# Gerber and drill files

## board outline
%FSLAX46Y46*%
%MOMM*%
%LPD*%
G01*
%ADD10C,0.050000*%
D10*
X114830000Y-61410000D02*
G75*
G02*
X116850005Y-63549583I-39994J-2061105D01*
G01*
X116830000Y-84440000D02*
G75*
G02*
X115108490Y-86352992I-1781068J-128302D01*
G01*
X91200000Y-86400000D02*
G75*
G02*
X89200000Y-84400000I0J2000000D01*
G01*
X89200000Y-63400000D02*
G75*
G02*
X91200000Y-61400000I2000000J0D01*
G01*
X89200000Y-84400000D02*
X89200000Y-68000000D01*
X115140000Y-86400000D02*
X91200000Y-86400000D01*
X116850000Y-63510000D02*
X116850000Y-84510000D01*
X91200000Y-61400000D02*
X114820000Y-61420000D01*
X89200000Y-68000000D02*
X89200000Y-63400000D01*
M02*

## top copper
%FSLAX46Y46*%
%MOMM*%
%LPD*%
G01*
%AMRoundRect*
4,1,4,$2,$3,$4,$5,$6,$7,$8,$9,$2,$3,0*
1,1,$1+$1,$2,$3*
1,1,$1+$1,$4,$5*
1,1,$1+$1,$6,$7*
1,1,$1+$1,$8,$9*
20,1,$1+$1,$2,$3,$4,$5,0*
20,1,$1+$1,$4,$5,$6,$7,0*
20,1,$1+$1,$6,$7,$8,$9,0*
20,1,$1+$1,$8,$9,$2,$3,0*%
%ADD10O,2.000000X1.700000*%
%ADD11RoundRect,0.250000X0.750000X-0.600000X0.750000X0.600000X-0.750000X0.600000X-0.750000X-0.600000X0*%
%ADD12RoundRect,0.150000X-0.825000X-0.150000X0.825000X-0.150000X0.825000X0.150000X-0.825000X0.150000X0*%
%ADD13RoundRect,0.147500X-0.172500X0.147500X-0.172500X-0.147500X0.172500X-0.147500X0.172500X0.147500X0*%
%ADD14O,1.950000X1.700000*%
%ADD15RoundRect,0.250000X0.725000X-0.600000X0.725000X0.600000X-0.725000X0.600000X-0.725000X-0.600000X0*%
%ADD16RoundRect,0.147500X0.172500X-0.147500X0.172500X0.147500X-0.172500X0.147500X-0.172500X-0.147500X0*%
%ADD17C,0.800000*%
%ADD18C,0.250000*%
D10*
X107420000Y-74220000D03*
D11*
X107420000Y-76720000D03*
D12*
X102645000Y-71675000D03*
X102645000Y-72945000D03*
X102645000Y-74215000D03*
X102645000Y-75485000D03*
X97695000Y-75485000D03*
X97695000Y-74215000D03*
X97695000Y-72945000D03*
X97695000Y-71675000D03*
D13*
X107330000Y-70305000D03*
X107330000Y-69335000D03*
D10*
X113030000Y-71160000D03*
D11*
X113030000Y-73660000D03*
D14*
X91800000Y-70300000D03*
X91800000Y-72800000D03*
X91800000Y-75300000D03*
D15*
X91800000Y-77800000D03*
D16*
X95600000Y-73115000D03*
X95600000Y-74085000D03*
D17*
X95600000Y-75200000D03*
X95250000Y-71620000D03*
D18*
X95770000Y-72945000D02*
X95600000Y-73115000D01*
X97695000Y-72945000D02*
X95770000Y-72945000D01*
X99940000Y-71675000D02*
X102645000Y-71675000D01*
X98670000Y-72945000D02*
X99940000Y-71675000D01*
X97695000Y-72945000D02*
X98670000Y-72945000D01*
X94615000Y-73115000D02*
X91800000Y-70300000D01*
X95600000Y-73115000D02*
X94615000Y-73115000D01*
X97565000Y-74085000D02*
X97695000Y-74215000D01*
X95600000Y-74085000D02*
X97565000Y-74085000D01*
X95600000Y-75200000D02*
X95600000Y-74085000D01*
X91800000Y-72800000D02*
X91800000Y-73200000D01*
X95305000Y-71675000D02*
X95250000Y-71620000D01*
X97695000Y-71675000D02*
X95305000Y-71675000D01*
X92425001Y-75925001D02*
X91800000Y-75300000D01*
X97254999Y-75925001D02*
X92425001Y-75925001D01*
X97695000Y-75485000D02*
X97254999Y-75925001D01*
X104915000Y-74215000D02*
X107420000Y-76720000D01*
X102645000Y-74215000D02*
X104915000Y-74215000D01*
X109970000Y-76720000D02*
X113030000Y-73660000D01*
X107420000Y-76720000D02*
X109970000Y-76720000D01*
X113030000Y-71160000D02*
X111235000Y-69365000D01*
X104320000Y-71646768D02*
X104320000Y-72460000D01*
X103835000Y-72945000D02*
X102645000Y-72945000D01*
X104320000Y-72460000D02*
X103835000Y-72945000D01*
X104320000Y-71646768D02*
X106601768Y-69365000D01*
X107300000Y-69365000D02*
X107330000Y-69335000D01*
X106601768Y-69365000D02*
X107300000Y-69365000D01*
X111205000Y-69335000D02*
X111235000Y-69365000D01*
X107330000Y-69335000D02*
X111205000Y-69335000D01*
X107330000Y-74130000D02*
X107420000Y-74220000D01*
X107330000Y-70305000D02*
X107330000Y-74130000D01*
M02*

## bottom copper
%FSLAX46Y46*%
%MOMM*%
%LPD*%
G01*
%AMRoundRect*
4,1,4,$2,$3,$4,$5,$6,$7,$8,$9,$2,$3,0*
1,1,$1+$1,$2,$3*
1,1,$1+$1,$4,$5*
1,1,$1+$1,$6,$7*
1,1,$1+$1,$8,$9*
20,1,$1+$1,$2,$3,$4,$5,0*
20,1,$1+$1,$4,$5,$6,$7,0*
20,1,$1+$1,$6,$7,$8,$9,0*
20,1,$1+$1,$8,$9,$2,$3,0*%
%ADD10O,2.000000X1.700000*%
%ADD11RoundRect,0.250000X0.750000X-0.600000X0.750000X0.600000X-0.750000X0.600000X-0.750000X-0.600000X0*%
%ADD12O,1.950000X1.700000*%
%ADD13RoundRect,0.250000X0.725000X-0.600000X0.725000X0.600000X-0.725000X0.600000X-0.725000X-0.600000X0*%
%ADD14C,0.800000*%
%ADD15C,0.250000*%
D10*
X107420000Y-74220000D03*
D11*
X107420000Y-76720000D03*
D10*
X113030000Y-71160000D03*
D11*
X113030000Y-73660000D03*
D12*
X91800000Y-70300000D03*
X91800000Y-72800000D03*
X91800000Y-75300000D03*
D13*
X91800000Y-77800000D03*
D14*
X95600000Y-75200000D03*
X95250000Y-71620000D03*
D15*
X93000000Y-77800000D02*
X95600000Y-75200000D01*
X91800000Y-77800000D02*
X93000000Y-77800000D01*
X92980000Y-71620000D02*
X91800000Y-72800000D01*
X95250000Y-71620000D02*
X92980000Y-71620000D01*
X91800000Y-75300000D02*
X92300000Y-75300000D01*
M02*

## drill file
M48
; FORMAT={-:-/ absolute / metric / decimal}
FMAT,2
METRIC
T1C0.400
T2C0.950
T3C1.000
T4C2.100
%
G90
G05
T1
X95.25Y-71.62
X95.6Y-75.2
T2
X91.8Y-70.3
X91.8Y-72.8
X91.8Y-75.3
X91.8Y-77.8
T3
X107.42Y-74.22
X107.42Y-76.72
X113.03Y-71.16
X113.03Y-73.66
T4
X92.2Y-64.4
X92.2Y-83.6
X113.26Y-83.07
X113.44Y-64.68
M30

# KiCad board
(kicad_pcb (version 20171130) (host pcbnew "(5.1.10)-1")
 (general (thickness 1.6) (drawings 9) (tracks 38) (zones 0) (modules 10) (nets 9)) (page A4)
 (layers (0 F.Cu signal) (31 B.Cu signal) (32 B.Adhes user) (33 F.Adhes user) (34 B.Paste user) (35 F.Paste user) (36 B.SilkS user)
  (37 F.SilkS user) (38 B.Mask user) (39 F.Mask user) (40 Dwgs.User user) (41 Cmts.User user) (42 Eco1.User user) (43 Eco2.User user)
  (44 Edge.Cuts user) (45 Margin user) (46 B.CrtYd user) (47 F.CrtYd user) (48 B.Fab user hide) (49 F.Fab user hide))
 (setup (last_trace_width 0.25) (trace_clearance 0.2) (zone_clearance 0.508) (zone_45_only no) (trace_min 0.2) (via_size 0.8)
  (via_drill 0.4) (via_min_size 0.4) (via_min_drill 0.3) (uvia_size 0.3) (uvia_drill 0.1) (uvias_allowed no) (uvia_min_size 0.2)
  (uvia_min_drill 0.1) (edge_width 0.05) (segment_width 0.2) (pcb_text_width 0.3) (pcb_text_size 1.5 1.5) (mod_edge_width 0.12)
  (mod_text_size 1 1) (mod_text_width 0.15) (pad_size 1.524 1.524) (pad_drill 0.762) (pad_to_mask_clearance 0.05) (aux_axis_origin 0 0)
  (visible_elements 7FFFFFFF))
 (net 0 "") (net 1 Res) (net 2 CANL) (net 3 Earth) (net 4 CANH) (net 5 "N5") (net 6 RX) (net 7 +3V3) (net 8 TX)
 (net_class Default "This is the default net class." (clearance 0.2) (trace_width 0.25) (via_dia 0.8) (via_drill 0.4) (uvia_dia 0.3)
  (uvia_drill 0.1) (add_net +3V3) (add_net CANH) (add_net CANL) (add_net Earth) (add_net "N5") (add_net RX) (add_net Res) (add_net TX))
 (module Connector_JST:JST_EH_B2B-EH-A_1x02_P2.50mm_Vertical (layer F.Cu) (at 107.42 76.72 90)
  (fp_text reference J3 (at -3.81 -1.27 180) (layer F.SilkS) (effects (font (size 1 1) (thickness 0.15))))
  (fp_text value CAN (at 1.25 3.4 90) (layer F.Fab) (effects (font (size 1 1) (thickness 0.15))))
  (pad 2 thru_hole oval (at 2.5 0 90) (size 1.7 2) (drill 1) (layers *.Cu *.Mask) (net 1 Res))
  (pad 1 thru_hole roundrect (at 0 0 90) (size 1.7 2) (drill 1) (layers *.Cu *.Mask) (roundrect_rratio 0.147059) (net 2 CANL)))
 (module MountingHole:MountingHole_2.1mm (layer F.Cu) (at 113.26 83.07)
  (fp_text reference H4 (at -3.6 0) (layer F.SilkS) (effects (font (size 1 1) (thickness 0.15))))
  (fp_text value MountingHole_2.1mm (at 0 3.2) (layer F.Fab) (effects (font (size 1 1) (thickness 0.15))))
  (pad "" np_thru_hole circle (at 0 0) (size 2.1 2.1) (drill 2.1) (layers *.Cu *.Mask)))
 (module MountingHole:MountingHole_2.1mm (layer F.Cu) (at 92.2 83.6)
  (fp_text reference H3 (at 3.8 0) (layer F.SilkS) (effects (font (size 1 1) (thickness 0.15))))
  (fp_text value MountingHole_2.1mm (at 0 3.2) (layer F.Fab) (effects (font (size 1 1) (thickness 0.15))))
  (pad "" np_thru_hole circle (at 0 0) (size 2.1 2.1) (drill 2.1) (layers *.Cu *.Mask)))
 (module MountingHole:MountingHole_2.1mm (layer F.Cu) (at 113.44 64.68)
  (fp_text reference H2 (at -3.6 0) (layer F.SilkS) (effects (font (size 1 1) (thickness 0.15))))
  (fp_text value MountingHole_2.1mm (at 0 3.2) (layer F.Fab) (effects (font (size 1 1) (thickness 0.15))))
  (pad "" np_thru_hole circle (at 0 0) (size 2.1 2.1) (drill 2.1) (layers *.Cu *.Mask)))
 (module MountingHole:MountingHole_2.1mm (layer F.Cu) (at 92.2 64.4)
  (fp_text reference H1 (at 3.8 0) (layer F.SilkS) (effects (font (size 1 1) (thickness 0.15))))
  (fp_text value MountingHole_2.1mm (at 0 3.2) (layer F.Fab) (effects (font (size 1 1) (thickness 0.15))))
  (pad "" np_thru_hole circle (at 0 0) (size 2.1 2.1) (drill 2.1) (layers *.Cu *.Mask)))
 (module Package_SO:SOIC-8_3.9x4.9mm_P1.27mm (layer F.Cu) (at 100.17 73.58)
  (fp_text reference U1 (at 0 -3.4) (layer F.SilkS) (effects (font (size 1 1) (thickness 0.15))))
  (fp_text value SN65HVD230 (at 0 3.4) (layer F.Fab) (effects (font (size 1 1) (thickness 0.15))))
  (pad 8 smd roundrect (at 2.475 -1.905) (size 1.95 0.6) (layers F.Cu F.Paste F.Mask) (roundrect_rratio 0.25) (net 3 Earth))
  (pad 7 smd roundrect (at 2.475 -0.635) (size 1.95 0.6) (layers F.Cu F.Paste F.Mask) (roundrect_rratio 0.25) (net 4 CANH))
  (pad 6 smd roundrect (at 2.475 0.635) (size 1.95 0.6) (layers F.Cu F.Paste F.Mask) (roundrect_rratio 0.25) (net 2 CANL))
  (pad 5 smd roundrect (at 2.475 1.905) (size 1.95 0.6) (layers F.Cu F.Paste F.Mask) (roundrect_rratio 0.25) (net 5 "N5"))
  (pad 4 smd roundrect (at -2.475 1.905) (size 1.95 0.6) (layers F.Cu F.Paste F.Mask) (roundrect_rratio 0.25) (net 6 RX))
  (pad 3 smd roundrect (at -2.475 0.635) (size 1.95 0.6) (layers F.Cu F.Paste F.Mask) (roundrect_rratio 0.25) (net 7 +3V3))
  (pad 2 smd roundrect (at -2.475 -0.635) (size 1.95 0.6) (layers F.Cu F.Paste F.Mask) (roundrect_rratio 0.25) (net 3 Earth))
  (pad 1 smd roundrect (at -2.475 -1.905) (size 1.95 0.6) (layers F.Cu F.Paste F.Mask) (roundrect_rratio 0.25) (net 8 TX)))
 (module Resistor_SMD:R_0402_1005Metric (layer F.Cu) (at 107.33 69.82 270)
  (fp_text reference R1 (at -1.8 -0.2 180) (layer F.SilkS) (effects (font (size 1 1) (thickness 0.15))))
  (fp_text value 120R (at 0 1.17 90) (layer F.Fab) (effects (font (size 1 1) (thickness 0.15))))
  (pad 2 smd roundrect (at 0.485 0 270) (size 0.59 0.64) (layers F.Cu F.Paste F.Mask) (roundrect_rratio 0.25) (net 1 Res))
  (pad 1 smd roundrect (at -0.485 0 270) (size 0.59 0.64) (layers F.Cu F.Paste F.Mask) (roundrect_rratio 0.25) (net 4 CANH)))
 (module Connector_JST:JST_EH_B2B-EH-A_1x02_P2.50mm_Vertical (layer F.Cu) (at 113.03 73.66 90)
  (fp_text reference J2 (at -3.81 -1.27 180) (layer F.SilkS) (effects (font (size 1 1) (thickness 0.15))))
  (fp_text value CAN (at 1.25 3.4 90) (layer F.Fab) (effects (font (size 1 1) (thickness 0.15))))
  (pad 2 thru_hole oval (at 2.5 0 90) (size 1.7 2) (drill 1) (layers *.Cu *.Mask) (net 4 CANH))
  (pad 1 thru_hole roundrect (at 0 0 90) (size 1.7 2) (drill 1) (layers *.Cu *.Mask) (roundrect_rratio 0.147059) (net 2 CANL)))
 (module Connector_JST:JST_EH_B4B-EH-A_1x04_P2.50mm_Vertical (layer F.Cu) (at 91.8 77.8 90)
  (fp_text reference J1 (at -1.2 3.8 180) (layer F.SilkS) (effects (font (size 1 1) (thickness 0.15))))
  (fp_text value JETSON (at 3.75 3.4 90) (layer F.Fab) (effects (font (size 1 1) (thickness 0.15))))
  (pad 4 thru_hole oval (at 7.5 0 90) (size 1.7 1.95) (drill 0.95) (layers *.Cu *.Mask) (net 3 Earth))
  (pad 3 thru_hole oval (at 5 0 90) (size 1.7 1.95) (drill 0.95) (layers *.Cu *.Mask) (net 8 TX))
  (pad 2 thru_hole oval (at 2.5 0 90) (size 1.7 1.95) (drill 0.95) (layers *.Cu *.Mask) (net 6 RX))
  (pad 1 thru_hole roundrect (at 0 0 90) (size 1.7 1.95) (drill 0.95) (layers *.Cu *.Mask) (roundrect_rratio 0.147059) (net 7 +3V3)))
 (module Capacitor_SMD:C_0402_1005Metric (layer F.Cu) (at 95.6 73.6 90)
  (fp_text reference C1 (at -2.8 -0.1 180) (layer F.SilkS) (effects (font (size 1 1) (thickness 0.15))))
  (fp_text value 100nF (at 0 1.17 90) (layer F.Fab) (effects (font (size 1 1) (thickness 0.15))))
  (pad 2 smd roundrect (at 0.485 0 90) (size 0.59 0.64) (layers F.Cu F.Paste F.Mask) (roundrect_rratio 0.25) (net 3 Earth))
  (pad 1 smd roundrect (at -0.485 0 90) (size 0.59 0.64) (layers F.Cu F.Paste F.Mask) (roundrect_rratio 0.25) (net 7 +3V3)))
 (gr_arc (start 114.790006 63.471105) (end 116.850005 63.549583) (angle -91.07006917) (layer Edge.Cuts) (width 0.05))
 (gr_arc (start 115.048932 84.568302) (end 115.10849 86.352992) (angle -92.20892931) (layer Edge.Cuts) (width 0.05))
 (gr_arc (start 91.2 84.4) (end 89.2 84.4) (angle -90) (layer Edge.Cuts) (width 0.05))
 (gr_arc (start 91.2 63.4) (end 91.2 61.4) (angle -90) (layer Edge.Cuts) (width 0.05))
 (gr_line (start 89.2 84.4) (end 89.2 68) (layer Edge.Cuts) (width 0.05))
 (gr_line (start 115.14 86.4) (end 91.2 86.4) (layer Edge.Cuts) (width 0.05))
 (gr_line (start 116.85 63.51) (end 116.85 84.51) (layer Edge.Cuts) (width 0.05))
 (gr_line (start 91.2 61.4) (end 114.82 61.42) (layer Edge.Cuts) (width 0.05))
 (gr_line (start 89.2 68) (end 89.2 63.4) (layer Edge.Cuts) (width 0.05))
 (segment (start 95.77 72.945) (end 95.6 73.115) (width 0.25) (layer F.Cu) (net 3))
 (segment (start 97.695 72.945) (end 95.77 72.945) (width 0.25) (layer F.Cu) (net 3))
 (segment (start 99.94 71.675) (end 102.645 71.675) (width 0.25) (layer F.Cu) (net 3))
 (segment (start 98.67 72.945) (end 99.94 71.675) (width 0.25) (layer F.Cu) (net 3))
 (segment (start 97.695 72.945) (end 98.67 72.945) (width 0.25) (layer F.Cu) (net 3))
 (segment (start 94.615 73.115) (end 91.8 70.3) (width 0.25) (layer F.Cu) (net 3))
 (segment (start 95.6 73.115) (end 94.615 73.115) (width 0.25) (layer F.Cu) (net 3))
 (via (at 95.6 75.2) (size 0.8) (drill 0.4) (layers F.Cu B.Cu) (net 7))
 (segment (start 93 77.8) (end 95.6 75.2) (width 0.25) (layer B.Cu) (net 7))
 (segment (start 91.8 77.8) (end 93 77.8) (width 0.25) (layer B.Cu) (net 7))
 (segment (start 97.565 74.085) (end 97.695 74.215) (width 0.25) (layer F.Cu) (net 7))
 (segment (start 95.6 74.085) (end 97.565 74.085) (width 0.25) (layer F.Cu) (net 7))
 (segment (start 95.6 75.2) (end 95.6 74.085) (width 0.25) (layer F.Cu) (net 7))
 (via (at 95.25 71.62) (size 0.8) (drill 0.4) (layers F.Cu B.Cu) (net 8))
 (segment (start 91.8 72.8) (end 91.8 73.2) (width 0.25) (layer F.Cu) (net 8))
 (segment (start 95.305 71.675) (end 95.25 71.62) (width 0.25) (layer F.Cu) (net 8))
 (segment (start 97.695 71.675) (end 95.305 71.675) (width 0.25) (layer F.Cu) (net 8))
 (segment (start 92.98 71.62) (end 91.8 72.8) (width 0.25) (layer B.Cu) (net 8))
 (segment (start 95.25 71.62) (end 92.98 71.62) (width 0.25) (layer B.Cu) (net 8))
 (segment (start 91.8 75.3) (end 92.3 75.3) (width 0.25) (layer B.Cu) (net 6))
 (segment (start 92.425001 75.925001) (end 91.8 75.3) (width 0.25) (layer F.Cu) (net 6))
 (segment (start 97.254999 75.925001) (end 92.425001 75.925001) (width 0.25) (layer F.Cu) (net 6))
 (segment (start 97.695 75.485) (end 97.254999 75.925001) (width 0.25) (layer F.Cu) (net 6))
 (segment (start 104.915 74.215) (end 107.42 76.72) (width 0.25) (layer F.Cu) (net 2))
 (segment (start 102.645 74.215) (end 104.915 74.215) (width 0.25) (layer F.Cu) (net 2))
 (segment (start 109.97 76.72) (end 113.03 73.66) (width 0.25) (layer F.Cu) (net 2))
 (segment (start 107.42 76.72) (end 109.97 76.72) (width 0.25) (layer F.Cu) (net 2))
 (segment (start 113.03 71.16) (end 111.235 69.365) (width 0.25) (layer F.Cu) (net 4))
 (segment (start 104.32 71.646768) (end 104.32 72.46) (width 0.25) (layer F.Cu) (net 4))
 (segment (start 103.835 72.945) (end 102.645 72.945) (width 0.25) (layer F.Cu) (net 4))
 (segment (start 104.32 72.46) (end 103.835 72.945) (width 0.25) (layer F.Cu) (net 4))
 (segment (start 104.32 71.646768) (end 106.601768 69.365) (width 0.25) (layer F.Cu) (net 4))
 (segment (start 107.3 69.365) (end 107.33 69.335) (width 0.25) (layer F.Cu) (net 4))
 (segment (start 106.601768 69.365) (end 107.3 69.365) (width 0.25) (layer F.Cu) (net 4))
 (segment (start 111.205 69.335) (end 111.235 69.365) (width 0.25) (layer F.Cu) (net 4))
 (segment (start 107.33 69.335) (end 111.205 69.335) (width 0.25) (layer F.Cu) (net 4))
 (segment (start 107.33 74.13) (end 107.42 74.22) (width 0.25) (layer F.Cu) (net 1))
 (segment (start 107.33 70.305) (end 107.33 74.13) (width 0.25) (layer F.Cu) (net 1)))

